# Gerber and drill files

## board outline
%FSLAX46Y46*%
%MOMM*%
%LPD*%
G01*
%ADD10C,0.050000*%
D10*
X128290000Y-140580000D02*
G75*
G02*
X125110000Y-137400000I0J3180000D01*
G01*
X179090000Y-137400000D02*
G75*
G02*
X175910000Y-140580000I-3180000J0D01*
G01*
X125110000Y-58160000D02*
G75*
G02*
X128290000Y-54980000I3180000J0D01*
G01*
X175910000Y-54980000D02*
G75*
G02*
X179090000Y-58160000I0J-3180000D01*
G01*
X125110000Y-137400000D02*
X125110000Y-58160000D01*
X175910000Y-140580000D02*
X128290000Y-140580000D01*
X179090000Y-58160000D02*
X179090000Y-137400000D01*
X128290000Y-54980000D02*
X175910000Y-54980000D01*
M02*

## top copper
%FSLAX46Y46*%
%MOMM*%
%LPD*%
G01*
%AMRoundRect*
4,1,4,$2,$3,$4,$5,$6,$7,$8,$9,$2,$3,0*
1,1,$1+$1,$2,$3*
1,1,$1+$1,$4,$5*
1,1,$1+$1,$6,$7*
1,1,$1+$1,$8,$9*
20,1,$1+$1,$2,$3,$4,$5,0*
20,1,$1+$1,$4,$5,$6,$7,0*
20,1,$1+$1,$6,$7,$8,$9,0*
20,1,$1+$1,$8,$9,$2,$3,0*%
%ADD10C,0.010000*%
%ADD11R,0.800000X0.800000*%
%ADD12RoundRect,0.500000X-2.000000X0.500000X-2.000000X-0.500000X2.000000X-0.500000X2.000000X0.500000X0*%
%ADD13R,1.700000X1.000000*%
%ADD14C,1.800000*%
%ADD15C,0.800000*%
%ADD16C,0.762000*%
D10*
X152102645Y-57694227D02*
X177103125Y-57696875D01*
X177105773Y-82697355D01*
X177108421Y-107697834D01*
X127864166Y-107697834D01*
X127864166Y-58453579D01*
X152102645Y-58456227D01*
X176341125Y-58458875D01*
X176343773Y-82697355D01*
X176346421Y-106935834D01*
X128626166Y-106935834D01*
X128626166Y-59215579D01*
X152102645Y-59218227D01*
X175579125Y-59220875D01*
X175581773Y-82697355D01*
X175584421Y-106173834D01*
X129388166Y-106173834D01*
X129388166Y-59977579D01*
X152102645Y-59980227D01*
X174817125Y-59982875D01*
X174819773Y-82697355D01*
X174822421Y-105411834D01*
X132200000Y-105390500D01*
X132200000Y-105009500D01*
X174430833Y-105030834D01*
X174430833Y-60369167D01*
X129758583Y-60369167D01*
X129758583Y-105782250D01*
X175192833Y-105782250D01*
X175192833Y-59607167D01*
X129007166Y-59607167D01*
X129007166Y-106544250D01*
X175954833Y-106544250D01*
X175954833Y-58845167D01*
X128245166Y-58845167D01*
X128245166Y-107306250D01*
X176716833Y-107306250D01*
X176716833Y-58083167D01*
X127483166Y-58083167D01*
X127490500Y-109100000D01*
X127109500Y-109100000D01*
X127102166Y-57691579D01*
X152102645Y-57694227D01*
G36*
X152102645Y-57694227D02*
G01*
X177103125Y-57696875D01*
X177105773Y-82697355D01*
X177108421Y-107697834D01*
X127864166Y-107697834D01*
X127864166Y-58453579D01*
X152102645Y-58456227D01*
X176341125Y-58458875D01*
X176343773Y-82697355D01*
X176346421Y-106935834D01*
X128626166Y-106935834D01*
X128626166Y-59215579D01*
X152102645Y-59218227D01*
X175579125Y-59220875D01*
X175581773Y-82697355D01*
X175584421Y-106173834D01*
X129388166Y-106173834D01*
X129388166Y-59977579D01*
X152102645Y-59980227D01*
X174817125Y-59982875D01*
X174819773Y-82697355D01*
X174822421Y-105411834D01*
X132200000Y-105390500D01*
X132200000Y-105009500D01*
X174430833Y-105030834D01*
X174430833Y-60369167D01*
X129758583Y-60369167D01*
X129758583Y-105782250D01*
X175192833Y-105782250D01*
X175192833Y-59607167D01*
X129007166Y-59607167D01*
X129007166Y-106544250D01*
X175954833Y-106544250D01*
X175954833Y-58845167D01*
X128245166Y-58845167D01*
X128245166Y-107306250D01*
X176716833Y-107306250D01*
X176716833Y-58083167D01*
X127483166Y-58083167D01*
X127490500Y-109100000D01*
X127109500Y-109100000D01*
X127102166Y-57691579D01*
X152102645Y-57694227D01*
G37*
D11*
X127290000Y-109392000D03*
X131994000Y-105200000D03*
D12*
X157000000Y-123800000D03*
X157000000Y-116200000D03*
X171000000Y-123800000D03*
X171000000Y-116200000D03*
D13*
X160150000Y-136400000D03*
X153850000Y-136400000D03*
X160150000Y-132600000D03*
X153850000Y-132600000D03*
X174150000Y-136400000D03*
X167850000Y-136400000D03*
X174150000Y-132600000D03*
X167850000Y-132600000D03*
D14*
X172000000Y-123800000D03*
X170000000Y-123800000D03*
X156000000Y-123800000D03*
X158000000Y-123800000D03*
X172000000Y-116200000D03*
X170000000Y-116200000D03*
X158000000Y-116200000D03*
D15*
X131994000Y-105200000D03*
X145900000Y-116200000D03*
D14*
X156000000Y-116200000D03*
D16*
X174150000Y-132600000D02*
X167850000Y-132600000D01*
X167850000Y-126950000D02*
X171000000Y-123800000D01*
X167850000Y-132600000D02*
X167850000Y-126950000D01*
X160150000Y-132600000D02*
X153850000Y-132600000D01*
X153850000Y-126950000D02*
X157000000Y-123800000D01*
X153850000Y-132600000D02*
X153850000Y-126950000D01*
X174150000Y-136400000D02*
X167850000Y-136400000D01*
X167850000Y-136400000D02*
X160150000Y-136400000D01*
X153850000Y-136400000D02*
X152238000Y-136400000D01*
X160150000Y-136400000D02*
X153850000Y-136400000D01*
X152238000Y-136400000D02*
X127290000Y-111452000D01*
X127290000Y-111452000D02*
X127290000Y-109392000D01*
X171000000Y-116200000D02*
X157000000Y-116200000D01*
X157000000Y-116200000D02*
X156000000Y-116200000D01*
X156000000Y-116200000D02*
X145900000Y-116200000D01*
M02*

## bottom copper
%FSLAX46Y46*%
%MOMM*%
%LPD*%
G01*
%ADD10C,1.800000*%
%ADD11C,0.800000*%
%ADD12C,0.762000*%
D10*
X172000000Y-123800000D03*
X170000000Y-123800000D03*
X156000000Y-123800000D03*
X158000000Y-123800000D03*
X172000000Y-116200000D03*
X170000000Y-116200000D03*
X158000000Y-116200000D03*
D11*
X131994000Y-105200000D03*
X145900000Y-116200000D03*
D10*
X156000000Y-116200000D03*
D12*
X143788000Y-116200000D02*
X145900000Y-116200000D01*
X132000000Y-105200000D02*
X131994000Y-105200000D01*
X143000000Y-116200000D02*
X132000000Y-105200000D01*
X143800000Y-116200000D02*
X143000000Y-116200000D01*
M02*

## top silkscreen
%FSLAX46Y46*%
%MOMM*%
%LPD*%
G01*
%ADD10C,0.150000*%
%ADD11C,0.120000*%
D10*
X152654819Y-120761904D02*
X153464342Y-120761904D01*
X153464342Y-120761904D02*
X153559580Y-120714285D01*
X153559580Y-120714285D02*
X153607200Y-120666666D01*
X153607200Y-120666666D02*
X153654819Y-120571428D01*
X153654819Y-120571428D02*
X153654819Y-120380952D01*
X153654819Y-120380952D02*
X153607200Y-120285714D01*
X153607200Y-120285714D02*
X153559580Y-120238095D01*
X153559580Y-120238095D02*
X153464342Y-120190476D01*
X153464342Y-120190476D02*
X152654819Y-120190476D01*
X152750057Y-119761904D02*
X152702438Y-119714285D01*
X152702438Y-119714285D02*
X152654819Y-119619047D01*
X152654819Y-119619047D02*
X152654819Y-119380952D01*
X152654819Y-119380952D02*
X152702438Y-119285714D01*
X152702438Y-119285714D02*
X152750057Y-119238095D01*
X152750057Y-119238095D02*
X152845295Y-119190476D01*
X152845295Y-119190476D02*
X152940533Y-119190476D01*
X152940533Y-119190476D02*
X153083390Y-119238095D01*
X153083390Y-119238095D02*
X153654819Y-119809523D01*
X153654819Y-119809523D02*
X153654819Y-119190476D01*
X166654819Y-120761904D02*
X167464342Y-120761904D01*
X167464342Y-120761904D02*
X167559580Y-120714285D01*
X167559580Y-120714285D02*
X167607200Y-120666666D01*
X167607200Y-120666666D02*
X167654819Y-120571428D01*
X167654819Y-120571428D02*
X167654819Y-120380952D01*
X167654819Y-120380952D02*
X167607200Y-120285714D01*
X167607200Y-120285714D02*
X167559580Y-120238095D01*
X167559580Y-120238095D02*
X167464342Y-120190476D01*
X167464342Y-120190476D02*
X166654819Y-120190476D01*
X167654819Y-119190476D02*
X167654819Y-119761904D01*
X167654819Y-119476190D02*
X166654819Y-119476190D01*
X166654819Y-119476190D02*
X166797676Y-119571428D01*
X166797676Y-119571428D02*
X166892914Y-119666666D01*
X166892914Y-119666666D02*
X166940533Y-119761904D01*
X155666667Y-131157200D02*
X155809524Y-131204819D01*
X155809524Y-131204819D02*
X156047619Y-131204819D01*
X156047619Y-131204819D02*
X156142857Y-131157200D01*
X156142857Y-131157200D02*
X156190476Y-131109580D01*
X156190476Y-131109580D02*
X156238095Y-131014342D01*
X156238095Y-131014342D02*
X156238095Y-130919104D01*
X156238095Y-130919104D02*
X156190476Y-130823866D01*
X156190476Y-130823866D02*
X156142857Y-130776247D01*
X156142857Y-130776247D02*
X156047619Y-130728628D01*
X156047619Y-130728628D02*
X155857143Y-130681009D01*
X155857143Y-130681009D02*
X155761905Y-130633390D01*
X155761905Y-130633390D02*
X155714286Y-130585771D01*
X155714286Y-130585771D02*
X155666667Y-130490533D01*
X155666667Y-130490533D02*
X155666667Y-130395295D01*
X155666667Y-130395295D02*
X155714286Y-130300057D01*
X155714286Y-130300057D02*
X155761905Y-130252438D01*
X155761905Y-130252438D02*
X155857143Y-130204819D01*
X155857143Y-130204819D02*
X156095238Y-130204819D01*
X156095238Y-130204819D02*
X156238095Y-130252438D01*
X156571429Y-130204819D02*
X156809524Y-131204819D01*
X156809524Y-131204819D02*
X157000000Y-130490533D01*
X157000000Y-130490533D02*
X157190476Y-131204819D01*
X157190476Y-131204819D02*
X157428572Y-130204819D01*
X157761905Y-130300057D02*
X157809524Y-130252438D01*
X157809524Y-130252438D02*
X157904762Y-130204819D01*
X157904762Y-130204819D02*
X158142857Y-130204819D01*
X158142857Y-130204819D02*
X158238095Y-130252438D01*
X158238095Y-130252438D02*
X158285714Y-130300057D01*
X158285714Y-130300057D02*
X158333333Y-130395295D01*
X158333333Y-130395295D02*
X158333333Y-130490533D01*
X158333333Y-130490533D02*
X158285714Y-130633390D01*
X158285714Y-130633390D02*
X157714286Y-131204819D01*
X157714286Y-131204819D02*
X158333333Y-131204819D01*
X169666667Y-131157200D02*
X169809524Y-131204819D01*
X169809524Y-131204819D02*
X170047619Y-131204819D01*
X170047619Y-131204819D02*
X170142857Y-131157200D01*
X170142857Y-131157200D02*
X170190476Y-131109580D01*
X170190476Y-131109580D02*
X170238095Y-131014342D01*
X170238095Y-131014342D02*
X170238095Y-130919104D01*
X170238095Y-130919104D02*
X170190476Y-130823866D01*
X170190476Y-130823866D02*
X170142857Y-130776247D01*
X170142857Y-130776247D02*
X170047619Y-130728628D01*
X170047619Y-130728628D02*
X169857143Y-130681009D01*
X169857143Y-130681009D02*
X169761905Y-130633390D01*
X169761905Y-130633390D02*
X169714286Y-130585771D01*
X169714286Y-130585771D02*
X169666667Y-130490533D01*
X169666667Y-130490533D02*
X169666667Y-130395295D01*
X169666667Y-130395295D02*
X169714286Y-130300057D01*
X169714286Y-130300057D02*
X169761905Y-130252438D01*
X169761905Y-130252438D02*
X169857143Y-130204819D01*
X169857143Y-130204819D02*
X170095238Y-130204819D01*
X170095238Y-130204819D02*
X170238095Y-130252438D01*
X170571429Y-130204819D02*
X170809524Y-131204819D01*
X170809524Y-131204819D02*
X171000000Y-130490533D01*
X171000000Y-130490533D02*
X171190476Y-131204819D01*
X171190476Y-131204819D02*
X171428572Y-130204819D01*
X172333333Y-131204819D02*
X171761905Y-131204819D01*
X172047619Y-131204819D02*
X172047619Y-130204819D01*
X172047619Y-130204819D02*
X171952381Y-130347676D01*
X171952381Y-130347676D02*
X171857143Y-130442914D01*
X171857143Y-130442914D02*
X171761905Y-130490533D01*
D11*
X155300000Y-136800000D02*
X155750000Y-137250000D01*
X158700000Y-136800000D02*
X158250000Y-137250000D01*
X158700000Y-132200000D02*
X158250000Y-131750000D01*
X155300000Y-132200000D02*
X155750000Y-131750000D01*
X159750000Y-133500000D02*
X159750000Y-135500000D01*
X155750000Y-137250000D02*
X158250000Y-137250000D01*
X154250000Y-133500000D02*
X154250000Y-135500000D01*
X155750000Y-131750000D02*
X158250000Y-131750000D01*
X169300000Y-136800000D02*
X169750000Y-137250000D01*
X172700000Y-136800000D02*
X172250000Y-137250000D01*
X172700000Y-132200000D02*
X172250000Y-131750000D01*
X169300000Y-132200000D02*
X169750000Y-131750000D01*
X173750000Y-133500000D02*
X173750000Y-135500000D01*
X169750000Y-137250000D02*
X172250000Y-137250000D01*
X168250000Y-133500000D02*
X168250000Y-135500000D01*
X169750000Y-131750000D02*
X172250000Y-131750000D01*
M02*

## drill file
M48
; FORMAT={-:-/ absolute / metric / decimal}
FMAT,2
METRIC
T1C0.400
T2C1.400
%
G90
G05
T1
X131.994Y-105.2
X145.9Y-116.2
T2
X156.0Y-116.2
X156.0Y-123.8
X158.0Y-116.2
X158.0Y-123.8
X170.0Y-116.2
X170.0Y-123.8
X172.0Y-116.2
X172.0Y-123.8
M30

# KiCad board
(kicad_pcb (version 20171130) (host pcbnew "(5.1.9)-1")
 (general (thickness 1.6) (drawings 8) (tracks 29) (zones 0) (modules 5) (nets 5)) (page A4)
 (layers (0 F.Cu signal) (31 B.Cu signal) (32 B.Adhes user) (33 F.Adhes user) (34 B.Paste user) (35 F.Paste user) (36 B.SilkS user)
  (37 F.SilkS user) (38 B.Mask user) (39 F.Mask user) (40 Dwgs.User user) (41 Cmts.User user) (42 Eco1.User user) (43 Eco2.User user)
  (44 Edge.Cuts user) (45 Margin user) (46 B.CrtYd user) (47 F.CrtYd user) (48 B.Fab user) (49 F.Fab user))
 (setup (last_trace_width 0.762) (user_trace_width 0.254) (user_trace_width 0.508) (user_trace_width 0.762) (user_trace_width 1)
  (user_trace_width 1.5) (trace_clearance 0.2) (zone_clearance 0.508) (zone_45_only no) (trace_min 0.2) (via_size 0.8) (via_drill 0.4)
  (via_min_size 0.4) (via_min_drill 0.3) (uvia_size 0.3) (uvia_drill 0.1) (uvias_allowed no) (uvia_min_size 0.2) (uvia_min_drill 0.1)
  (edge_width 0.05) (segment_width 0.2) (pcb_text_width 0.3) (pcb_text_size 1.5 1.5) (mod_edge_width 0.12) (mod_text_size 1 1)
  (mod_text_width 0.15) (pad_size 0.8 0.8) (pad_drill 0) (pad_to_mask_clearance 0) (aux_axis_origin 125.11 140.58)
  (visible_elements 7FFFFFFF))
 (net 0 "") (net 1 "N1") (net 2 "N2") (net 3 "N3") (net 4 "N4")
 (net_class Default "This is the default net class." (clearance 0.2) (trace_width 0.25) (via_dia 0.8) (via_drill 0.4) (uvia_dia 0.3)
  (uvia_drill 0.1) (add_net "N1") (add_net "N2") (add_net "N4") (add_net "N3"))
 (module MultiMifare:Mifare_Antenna (layer F.Cu) (at 152.1 82.7 90)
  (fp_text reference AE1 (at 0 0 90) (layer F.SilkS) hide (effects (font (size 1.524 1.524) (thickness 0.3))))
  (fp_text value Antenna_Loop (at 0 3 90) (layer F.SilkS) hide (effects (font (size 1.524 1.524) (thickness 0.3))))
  (fp_poly
   (pts (xy 25.005773 0.002645) (xy 25.003125 25.003125) (xy 0.002645 25.005773) (xy -24.997834 25.008421) (xy -24.997834 -24.235834)
    (xy 24.246421 -24.235834) (xy 24.243773 0.002645) (xy 24.241125 24.241125) (xy 0.002645 24.243773) (xy -24.235834 24.246421)
    (xy -24.235834 -23.473834) (xy 23.484421 -23.473834) (xy 23.481773 0.002645) (xy 23.479125 23.479125) (xy 0.002645 23.481773)
    (xy -23.473834 23.484421) (xy -23.473834 -22.711834) (xy 22.722421 -22.711834) (xy 22.719773 0.002645) (xy 22.717125 22.717125)
    (xy 0.002645 22.719773) (xy -22.711834 22.722421) (xy -22.6905 -19.9) (xy -22.3095 -19.9) (xy -22.330834 22.330833)
    (xy 22.330833 22.330833) (xy 22.330833 -22.341417) (xy -23.08225 -22.341417) (xy -23.08225 23.092833) (xy 23.092833 23.092833)
    (xy 23.092833 -23.092834) (xy -23.84425 -23.092834) (xy -23.84425 23.854833) (xy 23.854833 23.854833) (xy 23.854833 -23.854834)
    (xy -24.60625 -23.854834) (xy -24.60625 24.616833) (xy 24.616833 24.616833) (xy 24.616833 -24.616834) (xy -26.4 -24.6095)
    (xy -26.4 -24.9905) (xy 25.008421 -24.997834) (xy 25.005773 0.002645))
   (layer F.Cu) (width 0.01))
  (pad 1 smd rect (at -26.692 -24.81 90) (size 0.8 0.8) (layers F.Cu F.Paste F.Mask) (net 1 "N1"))
  (pad 2 smd rect (at -22.5 -20.106 90) (size 0.8 0.8) (layers F.Cu F.Paste F.Mask) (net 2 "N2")))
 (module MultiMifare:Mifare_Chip (layer F.Cu) (at 157 120 270)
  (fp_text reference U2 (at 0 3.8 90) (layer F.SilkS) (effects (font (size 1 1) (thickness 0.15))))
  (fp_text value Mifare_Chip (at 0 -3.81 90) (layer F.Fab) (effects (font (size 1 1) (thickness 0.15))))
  (pad 2 smd roundrect (at 3.8 0 270) (size 2 5) (layers F.Cu F.Paste F.Mask) (roundrect_rratio 0.25) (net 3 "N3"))
  (pad 1 smd roundrect (at -3.8 0 270) (size 2 5) (layers F.Cu F.Paste F.Mask) (roundrect_rratio 0.25) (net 2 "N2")))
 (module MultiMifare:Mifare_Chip (layer F.Cu) (at 171 120 270)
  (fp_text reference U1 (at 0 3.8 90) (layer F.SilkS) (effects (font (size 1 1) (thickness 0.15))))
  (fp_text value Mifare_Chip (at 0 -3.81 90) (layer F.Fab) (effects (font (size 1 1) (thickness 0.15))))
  (pad 2 smd roundrect (at 3.8 0 270) (size 2 5) (layers F.Cu F.Paste F.Mask) (roundrect_rratio 0.25) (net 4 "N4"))
  (pad 1 smd roundrect (at -3.8 0 270) (size 2 5) (layers F.Cu F.Paste F.Mask) (roundrect_rratio 0.25) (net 2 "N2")))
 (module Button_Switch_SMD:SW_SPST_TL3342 (layer F.Cu) (at 157 134.5)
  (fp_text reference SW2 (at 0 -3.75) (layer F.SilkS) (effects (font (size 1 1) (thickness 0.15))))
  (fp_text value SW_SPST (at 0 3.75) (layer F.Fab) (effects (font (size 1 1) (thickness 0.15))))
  (fp_line (start -1.7 2.3) (end -1.25 2.75) (layer F.SilkS) (width 0.12))
  (fp_line (start 1.7 2.3) (end 1.25 2.75) (layer F.SilkS) (width 0.12))
  (fp_line (start 1.7 -2.3) (end 1.25 -2.75) (layer F.SilkS) (width 0.12))
  (fp_line (start -1.7 -2.3) (end -1.25 -2.75) (layer F.SilkS) (width 0.12))
  (fp_line (start 2.75 -1) (end 2.75 1) (layer F.SilkS) (width 0.12))
  (fp_line (start -1.25 2.75) (end 1.25 2.75) (layer F.SilkS) (width 0.12))
  (fp_line (start -2.75 -1) (end -2.75 1) (layer F.SilkS) (width 0.12))
  (fp_line (start -1.25 -2.75) (end 1.25 -2.75) (layer F.SilkS) (width 0.12))
  (pad 2 smd rect (at 3.15 1.9) (size 1.7 1) (layers F.Cu F.Paste F.Mask) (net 1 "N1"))
  (pad 2 smd rect (at -3.15 1.9) (size 1.7 1) (layers F.Cu F.Paste F.Mask) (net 1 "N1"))
  (pad 1 smd rect (at 3.15 -1.9) (size 1.7 1) (layers F.Cu F.Paste F.Mask) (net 3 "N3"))
  (pad 1 smd rect (at -3.15 -1.9) (size 1.7 1) (layers F.Cu F.Paste F.Mask) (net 3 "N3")))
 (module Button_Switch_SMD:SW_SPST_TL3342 (layer F.Cu) (at 171 134.5)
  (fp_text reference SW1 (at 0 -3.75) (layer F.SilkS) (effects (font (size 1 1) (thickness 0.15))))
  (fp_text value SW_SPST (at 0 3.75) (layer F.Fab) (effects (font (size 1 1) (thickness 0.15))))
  (fp_line (start -1.7 2.3) (end -1.25 2.75) (layer F.SilkS) (width 0.12))
  (fp_line (start 1.7 2.3) (end 1.25 2.75) (layer F.SilkS) (width 0.12))
  (fp_line (start 1.7 -2.3) (end 1.25 -2.75) (layer F.SilkS) (width 0.12))
  (fp_line (start -1.7 -2.3) (end -1.25 -2.75) (layer F.SilkS) (width 0.12))
  (fp_line (start 2.75 -1) (end 2.75 1) (layer F.SilkS) (width 0.12))
  (fp_line (start -1.25 2.75) (end 1.25 2.75) (layer F.SilkS) (width 0.12))
  (fp_line (start -2.75 -1) (end -2.75 1) (layer F.SilkS) (width 0.12))
  (fp_line (start -1.25 -2.75) (end 1.25 -2.75) (layer F.SilkS) (width 0.12))
  (pad 2 smd rect (at 3.15 1.9) (size 1.7 1) (layers F.Cu F.Paste F.Mask) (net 1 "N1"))
  (pad 2 smd rect (at -3.15 1.9) (size 1.7 1) (layers F.Cu F.Paste F.Mask) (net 1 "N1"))
  (pad 1 smd rect (at 3.15 -1.9) (size 1.7 1) (layers F.Cu F.Paste F.Mask) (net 4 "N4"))
  (pad 1 smd rect (at -3.15 -1.9) (size 1.7 1) (layers F.Cu F.Paste F.Mask) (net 4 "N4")))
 (gr_arc (start 128.29 137.4) (end 125.11 137.4) (angle -90) (layer Edge.Cuts) (width 0.05))
 (gr_arc (start 175.91 137.4) (end 175.91 140.58) (angle -90) (layer Edge.Cuts) (width 0.05))
 (gr_arc (start 128.29 58.16) (end 128.29 54.98) (angle -90) (layer Edge.Cuts) (width 0.05))
 (gr_arc (start 175.91 58.16) (end 179.09 58.16) (angle -90) (layer Edge.Cuts) (width 0.05))
 (gr_line (start 125.11 137.4) (end 125.11 58.16) (layer Edge.Cuts) (width 0.05))
 (gr_line (start 175.91 140.58) (end 128.29 140.58) (layer Edge.Cuts) (width 0.05))
 (gr_line (start 179.09 58.16) (end 179.09 137.4) (layer Edge.Cuts) (width 0.05))
 (gr_line (start 128.29 54.98) (end 175.91 54.98) (layer Edge.Cuts) (width 0.05))
 (via (at 172 123.8) (size 1.8) (drill 1.4) (layers F.Cu B.Cu) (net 4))
 (via (at 170 123.8) (size 1.8) (drill 1.4) (layers F.Cu B.Cu) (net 4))
 (via (at 156 123.8) (size 1.8) (drill 1.4) (layers F.Cu B.Cu) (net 3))
 (via (at 158 123.8) (size 1.8) (drill 1.4) (layers F.Cu B.Cu) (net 3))
 (via (at 172 116.2) (size 1.8) (drill 1.4) (layers F.Cu B.Cu) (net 2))
 (via (at 170 116.2) (size 1.8) (drill 1.4) (layers F.Cu B.Cu) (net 2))
 (via (at 158 116.2) (size 1.8) (drill 1.4) (layers F.Cu B.Cu) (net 2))
 (segment (start 174.15 132.6) (end 167.85 132.6) (width 0.762) (layer F.Cu) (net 4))
 (segment (start 167.85 126.95) (end 171 123.8) (width 0.762) (layer F.Cu) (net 4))
 (segment (start 167.85 132.6) (end 167.85 126.95) (width 0.762) (layer F.Cu) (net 4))
 (segment (start 160.15 132.6) (end 153.85 132.6) (width 0.762) (layer F.Cu) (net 3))
 (segment (start 153.85 126.95) (end 157 123.8) (width 0.762) (layer F.Cu) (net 3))
 (segment (start 153.85 132.6) (end 153.85 126.95) (width 0.762) (layer F.Cu) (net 3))
 (segment (start 174.15 136.4) (end 167.85 136.4) (width 0.762) (layer F.Cu) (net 1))
 (segment (start 167.85 136.4) (end 160.15 136.4) (width 0.762) (layer F.Cu) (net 1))
 (segment (start 153.85 136.4) (end 152.238 136.4) (width 0.762) (layer F.Cu) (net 1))
 (segment (start 160.15 136.4) (end 153.85 136.4) (width 0.762) (layer F.Cu) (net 1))
 (segment (start 152.238 136.4) (end 127.29 111.452) (width 0.762) (layer F.Cu) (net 1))
 (segment (start 127.29 111.452) (end 127.29 109.392) (width 0.762) (layer F.Cu) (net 1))
 (via (at 131.994 105.2) (size 0.8) (drill 0.4) (layers F.Cu B.Cu) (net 2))
 (via (at 145.9 116.2) (size 0.8) (drill 0.4) (layers F.Cu B.Cu) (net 2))
 (segment (start 143.788 116.2) (end 145.9 116.2) (width 0.762) (layer B.Cu) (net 2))
 (segment (start 132 105.2) (end 131.994 105.2) (width 0.762) (layer B.Cu) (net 2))
 (segment (start 143 116.2) (end 132 105.2) (width 0.762) (layer B.Cu) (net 2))
 (segment (start 143.8 116.2) (end 143 116.2) (width 0.762) (layer B.Cu) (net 2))
 (segment (start 171 116.2) (end 157 116.2) (width 0.762) (layer F.Cu) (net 2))
 (segment (start 157 116.2) (end 156 116.2) (width 0.762) (layer F.Cu) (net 2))
 (segment (start 156 116.2) (end 145.9 116.2) (width 0.762) (layer F.Cu) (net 2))
 (via (at 156 116.2) (size 1.8) (drill 1.4) (layers F.Cu B.Cu) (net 2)))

